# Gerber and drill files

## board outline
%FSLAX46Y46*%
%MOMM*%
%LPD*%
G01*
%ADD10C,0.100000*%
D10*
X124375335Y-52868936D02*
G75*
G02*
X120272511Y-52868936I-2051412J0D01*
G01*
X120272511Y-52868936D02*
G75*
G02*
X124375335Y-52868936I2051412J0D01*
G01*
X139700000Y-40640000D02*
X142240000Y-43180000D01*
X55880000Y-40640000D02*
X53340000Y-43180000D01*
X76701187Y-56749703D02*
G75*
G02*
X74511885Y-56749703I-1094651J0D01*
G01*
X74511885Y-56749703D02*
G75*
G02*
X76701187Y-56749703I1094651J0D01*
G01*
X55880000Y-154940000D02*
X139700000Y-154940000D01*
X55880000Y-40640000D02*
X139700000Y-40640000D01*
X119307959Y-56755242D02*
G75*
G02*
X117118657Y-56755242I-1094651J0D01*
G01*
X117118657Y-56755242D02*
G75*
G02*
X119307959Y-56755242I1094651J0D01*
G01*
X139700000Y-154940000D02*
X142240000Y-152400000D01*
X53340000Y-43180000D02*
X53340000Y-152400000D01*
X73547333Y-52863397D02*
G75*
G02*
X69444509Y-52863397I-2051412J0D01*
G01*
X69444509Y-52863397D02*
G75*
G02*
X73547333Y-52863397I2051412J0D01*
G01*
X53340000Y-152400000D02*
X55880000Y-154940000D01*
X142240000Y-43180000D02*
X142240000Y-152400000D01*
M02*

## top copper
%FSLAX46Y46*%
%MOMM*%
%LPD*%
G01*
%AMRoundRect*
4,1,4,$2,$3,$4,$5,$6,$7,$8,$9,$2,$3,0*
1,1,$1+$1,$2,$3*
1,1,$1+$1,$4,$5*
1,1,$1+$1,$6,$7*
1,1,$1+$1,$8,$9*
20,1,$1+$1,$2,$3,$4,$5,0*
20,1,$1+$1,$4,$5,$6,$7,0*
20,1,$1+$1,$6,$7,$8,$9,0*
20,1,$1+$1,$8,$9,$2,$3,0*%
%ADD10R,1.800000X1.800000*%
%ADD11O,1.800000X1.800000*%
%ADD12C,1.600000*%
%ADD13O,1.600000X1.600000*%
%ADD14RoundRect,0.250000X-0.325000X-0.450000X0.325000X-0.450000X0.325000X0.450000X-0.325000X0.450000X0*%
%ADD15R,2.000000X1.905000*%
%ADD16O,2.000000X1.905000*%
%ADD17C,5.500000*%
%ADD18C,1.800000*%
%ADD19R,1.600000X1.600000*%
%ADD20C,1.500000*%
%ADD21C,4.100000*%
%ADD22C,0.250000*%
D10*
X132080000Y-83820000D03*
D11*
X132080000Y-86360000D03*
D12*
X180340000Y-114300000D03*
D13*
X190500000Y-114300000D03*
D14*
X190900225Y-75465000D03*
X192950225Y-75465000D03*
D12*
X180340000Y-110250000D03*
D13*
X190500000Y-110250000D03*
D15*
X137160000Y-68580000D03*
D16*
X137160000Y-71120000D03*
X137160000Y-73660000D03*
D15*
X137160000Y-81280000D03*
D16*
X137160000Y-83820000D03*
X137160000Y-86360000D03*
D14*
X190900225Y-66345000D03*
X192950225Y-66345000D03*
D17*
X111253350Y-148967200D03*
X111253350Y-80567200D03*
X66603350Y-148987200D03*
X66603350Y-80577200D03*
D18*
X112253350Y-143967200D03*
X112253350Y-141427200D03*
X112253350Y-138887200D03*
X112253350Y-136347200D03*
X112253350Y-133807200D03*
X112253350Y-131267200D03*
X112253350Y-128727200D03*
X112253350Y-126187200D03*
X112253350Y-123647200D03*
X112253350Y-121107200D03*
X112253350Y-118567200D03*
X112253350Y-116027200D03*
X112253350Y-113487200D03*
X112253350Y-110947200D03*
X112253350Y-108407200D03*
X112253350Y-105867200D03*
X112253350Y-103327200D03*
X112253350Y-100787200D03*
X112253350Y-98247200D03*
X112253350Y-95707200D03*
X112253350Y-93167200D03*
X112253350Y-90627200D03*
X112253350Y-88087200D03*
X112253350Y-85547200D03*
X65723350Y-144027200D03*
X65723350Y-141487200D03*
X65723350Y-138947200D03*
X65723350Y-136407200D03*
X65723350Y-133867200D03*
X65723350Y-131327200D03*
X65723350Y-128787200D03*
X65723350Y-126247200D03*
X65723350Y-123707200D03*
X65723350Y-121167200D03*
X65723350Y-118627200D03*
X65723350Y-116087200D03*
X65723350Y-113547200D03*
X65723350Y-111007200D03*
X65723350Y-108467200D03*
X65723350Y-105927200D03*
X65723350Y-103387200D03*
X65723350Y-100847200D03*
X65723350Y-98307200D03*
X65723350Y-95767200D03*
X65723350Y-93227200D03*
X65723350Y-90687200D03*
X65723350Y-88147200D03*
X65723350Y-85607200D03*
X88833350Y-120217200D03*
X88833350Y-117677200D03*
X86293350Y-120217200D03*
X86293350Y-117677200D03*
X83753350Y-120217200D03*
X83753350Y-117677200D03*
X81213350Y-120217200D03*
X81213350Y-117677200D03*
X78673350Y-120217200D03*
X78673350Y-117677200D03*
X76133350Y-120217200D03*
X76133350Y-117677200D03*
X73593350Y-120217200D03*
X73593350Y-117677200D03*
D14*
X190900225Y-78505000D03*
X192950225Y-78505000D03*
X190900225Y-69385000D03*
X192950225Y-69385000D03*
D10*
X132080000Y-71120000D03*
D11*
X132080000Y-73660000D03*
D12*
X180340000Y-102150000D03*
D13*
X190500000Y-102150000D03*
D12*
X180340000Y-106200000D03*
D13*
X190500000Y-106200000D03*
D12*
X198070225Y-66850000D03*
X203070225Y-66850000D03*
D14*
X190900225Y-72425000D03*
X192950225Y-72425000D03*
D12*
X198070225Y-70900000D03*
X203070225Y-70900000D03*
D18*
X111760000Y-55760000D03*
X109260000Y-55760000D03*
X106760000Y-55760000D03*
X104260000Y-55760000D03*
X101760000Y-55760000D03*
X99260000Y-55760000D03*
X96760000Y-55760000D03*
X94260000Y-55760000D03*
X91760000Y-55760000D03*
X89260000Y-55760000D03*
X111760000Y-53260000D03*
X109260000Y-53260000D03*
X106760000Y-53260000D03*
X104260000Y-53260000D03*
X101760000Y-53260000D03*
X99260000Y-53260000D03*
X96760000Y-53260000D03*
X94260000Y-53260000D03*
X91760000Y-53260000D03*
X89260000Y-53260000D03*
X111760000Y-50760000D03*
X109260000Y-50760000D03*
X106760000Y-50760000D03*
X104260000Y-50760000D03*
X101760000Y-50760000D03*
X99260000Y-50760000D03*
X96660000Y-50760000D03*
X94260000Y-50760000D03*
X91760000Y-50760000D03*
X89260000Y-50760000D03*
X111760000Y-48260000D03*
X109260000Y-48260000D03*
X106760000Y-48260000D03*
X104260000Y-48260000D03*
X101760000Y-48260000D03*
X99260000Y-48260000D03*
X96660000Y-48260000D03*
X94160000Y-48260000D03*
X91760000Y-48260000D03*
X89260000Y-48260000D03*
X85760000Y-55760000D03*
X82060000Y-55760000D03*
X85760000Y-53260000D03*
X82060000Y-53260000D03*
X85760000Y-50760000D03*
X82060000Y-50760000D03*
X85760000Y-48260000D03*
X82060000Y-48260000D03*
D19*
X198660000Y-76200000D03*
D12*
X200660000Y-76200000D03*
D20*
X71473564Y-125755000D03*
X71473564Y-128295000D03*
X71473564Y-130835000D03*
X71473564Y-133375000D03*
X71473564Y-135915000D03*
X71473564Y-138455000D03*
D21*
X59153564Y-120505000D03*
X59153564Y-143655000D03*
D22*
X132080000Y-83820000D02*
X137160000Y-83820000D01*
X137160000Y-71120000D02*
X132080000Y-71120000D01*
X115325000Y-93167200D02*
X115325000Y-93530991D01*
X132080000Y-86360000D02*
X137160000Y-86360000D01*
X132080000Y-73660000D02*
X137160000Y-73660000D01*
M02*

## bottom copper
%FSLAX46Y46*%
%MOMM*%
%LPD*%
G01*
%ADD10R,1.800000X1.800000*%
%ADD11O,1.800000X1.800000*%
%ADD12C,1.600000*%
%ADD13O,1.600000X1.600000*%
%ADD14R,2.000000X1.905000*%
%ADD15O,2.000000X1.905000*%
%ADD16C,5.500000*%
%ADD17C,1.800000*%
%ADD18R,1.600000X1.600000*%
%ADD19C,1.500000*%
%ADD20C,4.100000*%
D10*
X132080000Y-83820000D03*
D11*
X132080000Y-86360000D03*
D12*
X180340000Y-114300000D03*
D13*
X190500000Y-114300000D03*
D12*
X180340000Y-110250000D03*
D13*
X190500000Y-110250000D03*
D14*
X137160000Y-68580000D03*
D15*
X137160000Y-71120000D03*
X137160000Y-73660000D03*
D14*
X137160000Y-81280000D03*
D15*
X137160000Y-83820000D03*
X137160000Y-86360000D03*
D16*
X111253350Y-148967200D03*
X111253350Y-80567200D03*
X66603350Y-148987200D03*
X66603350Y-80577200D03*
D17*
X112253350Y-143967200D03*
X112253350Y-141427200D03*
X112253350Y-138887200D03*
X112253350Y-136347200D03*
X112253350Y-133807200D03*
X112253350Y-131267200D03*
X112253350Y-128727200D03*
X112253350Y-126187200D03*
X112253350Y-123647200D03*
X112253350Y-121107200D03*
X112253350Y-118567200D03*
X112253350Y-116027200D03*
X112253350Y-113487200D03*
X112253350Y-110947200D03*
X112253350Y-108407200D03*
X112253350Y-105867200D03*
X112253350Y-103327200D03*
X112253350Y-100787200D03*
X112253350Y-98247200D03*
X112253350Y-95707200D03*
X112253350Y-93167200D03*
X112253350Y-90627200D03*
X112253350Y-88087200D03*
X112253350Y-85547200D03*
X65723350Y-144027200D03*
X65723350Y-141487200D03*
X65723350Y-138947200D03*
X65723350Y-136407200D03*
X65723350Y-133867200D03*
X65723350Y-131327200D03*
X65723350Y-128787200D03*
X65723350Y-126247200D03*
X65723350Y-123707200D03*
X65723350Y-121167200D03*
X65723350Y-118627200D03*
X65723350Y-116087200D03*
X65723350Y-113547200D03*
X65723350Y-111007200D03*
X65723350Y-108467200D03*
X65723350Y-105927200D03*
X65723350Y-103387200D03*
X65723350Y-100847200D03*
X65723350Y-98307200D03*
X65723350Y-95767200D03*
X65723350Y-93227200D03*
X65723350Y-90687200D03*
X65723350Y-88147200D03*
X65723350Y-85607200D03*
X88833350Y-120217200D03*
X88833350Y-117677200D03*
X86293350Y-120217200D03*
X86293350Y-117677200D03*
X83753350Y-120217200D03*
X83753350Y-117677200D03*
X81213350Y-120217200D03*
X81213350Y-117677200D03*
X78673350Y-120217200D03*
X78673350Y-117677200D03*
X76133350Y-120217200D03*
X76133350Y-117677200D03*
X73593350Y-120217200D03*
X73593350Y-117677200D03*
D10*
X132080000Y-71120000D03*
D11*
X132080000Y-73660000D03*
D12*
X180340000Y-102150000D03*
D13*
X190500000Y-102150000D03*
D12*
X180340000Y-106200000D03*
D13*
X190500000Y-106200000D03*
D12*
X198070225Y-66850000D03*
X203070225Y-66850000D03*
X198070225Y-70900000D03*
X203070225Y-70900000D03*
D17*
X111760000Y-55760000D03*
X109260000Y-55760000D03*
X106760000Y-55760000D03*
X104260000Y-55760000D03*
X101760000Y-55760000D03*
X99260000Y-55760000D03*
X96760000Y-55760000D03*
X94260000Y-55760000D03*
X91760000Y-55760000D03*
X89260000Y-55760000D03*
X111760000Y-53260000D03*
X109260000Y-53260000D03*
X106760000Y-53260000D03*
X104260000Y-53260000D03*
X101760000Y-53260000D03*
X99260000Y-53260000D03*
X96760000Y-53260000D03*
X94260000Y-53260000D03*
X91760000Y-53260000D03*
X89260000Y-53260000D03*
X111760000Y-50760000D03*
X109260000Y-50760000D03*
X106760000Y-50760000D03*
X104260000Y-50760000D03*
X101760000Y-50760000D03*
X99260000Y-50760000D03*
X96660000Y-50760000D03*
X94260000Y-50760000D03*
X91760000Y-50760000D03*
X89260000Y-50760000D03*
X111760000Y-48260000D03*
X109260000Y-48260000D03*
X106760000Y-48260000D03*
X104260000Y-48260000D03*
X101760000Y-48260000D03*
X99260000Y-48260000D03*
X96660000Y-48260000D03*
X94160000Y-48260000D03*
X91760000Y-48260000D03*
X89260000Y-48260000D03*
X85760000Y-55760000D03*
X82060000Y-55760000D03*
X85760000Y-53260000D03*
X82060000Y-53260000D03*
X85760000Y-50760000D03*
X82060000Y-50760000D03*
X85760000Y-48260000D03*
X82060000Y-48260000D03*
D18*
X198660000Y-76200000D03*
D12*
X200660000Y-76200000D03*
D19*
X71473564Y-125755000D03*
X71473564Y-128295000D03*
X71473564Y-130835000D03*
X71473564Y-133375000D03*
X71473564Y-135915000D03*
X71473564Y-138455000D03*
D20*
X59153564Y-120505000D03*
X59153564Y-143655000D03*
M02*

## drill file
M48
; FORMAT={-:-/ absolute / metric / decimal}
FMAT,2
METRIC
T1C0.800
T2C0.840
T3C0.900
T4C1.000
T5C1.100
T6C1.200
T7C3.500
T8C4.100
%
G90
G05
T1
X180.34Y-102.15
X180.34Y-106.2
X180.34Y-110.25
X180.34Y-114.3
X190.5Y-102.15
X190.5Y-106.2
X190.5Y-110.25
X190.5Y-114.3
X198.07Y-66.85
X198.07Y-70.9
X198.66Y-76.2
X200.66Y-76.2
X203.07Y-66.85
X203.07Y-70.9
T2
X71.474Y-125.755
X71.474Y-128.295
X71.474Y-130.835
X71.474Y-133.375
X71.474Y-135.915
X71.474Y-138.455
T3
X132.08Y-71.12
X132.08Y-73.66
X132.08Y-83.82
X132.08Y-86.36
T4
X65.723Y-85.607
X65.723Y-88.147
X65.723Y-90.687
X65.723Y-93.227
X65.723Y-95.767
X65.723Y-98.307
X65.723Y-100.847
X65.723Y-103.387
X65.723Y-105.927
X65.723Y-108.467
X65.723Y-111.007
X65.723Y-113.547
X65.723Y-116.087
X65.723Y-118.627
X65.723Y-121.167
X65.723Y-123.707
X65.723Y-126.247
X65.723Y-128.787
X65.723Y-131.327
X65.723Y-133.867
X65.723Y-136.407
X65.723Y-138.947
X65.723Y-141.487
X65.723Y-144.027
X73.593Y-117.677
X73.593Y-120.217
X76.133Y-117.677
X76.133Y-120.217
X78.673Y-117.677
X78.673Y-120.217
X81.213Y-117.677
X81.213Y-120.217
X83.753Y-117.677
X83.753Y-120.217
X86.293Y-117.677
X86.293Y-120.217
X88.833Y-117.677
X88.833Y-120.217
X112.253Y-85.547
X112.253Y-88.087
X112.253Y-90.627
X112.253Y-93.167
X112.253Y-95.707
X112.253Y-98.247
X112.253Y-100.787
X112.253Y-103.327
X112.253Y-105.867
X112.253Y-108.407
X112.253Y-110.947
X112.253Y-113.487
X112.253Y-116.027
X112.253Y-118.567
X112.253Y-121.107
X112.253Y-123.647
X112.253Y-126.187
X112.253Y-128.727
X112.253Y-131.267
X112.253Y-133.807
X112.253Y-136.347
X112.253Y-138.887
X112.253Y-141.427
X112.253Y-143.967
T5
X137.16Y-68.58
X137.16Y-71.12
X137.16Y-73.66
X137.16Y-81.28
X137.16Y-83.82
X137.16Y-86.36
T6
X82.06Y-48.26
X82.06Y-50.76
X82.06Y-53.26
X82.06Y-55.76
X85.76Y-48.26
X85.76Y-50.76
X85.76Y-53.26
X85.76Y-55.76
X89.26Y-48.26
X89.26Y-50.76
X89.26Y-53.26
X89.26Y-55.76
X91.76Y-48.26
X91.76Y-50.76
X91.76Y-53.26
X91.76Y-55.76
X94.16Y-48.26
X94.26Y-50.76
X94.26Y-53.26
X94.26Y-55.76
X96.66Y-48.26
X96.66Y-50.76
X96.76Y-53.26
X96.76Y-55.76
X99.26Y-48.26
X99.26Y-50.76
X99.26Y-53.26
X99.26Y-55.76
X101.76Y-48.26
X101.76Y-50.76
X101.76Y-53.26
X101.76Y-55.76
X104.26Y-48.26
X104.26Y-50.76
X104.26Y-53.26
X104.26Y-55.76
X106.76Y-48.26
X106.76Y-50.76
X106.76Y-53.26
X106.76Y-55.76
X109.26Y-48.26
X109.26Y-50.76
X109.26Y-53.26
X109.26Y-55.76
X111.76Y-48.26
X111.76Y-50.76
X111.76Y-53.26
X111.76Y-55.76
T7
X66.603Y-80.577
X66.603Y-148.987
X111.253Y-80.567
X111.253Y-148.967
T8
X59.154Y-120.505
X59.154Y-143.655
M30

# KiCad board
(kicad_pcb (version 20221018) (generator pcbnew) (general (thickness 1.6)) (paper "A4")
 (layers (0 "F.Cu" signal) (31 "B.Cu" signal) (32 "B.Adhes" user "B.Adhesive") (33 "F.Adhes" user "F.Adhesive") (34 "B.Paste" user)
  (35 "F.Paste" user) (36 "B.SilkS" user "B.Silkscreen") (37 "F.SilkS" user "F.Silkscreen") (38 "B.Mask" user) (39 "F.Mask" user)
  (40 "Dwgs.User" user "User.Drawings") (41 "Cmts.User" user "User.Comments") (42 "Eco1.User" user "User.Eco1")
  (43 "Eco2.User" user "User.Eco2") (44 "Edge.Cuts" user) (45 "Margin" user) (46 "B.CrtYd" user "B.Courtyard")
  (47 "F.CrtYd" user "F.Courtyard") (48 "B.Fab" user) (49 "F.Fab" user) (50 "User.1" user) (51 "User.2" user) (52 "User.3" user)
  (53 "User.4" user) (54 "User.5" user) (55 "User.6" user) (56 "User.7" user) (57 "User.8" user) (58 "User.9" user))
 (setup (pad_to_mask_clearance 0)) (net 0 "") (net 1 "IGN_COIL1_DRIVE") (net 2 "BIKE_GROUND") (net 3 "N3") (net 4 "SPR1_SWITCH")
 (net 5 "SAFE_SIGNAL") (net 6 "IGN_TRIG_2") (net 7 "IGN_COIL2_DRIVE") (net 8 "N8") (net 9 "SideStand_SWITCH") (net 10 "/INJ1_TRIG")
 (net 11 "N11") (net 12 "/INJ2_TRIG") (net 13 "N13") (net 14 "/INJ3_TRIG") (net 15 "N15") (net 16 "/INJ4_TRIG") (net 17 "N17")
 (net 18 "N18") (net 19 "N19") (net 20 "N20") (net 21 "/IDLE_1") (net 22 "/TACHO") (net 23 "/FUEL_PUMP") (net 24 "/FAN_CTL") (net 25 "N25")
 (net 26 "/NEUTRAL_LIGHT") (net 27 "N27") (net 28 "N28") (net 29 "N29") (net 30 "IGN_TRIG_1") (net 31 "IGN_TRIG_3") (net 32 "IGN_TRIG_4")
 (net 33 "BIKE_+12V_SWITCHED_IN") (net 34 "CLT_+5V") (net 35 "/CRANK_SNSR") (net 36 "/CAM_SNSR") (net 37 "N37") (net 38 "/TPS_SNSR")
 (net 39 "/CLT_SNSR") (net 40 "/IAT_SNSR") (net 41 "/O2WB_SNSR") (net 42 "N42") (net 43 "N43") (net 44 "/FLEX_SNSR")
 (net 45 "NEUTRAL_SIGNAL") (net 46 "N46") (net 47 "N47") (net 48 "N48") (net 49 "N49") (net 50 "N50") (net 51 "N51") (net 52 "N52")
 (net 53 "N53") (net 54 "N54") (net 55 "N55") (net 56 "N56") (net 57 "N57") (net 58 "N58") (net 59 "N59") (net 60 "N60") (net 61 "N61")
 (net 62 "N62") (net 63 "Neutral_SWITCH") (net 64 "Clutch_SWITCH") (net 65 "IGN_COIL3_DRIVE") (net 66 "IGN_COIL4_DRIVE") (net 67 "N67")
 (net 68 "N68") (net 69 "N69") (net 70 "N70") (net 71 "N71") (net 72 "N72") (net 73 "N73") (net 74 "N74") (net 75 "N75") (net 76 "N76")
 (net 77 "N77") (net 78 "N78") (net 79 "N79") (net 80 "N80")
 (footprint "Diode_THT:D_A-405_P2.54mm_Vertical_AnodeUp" (layer "F.Cu") (at 132.08 83.82 -90)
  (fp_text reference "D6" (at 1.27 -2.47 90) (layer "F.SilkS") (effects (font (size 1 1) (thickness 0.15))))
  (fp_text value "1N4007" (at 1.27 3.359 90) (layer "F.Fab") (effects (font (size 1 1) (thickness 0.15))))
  (pad "1" thru_hole rect (at 0 0 270) (size 1.8 1.8) (drill 0.9) (layers "*.Cu" "*.Mask") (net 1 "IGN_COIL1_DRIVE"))
  (pad "2" thru_hole oval (at 2.54 0 270) (size 1.8 1.8) (drill 0.9) (layers "*.Cu" "*.Mask") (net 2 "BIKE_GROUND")))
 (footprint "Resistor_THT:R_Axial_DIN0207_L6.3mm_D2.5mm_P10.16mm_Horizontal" (layer "F.Cu") (at 180.34 114.3)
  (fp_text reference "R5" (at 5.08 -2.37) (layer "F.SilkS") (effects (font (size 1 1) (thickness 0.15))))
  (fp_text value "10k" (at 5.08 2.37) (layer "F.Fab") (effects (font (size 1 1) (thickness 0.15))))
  (pad "1" thru_hole circle (at 0 0) (size 1.6 1.6) (drill 0.8) (layers "*.Cu" "*.Mask") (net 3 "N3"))
  (pad "2" thru_hole oval (at 10.16 0) (size 1.6 1.6) (drill 0.8) (layers "*.Cu" "*.Mask") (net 2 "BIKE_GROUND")))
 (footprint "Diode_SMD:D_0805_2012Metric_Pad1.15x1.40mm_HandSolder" (layer "F.Cu") (at 191.925225 75.465)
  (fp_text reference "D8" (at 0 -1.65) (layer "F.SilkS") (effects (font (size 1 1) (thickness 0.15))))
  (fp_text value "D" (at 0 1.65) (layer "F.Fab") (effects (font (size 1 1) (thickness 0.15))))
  (pad "1" smd roundrect (at -1.025 0) (size 1.15 1.4) (layers "F.Cu" "F.Paste" "F.Mask") (roundrect_rratio 0.217391) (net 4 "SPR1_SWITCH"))
  (pad "2" smd roundrect (at 1.025 0) (size 1.15 1.4) (layers "F.Cu" "F.Paste" "F.Mask") (roundrect_rratio 0.217391) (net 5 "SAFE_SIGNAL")))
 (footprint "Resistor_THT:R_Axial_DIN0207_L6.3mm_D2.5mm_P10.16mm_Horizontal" (layer "F.Cu") (at 180.34 110.25)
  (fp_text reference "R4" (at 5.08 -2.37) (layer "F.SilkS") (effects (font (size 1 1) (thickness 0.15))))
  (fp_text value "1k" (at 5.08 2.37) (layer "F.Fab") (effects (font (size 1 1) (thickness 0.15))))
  (pad "1" thru_hole circle (at 0 0) (size 1.6 1.6) (drill 0.8) (layers "*.Cu" "*.Mask") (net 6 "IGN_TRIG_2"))
  (pad "2" thru_hole oval (at 10.16 0) (size 1.6 1.6) (drill 0.8) (layers "*.Cu" "*.Mask") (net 3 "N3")))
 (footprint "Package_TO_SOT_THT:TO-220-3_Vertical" (layer "F.Cu") (at 137.16 68.58 -90)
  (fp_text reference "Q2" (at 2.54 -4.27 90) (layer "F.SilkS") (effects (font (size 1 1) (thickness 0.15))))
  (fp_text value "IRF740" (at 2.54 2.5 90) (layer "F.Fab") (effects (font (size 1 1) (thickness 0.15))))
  (pad "1" thru_hole rect (at 0 0 270) (size 1.905 2) (drill 1.1) (layers "*.Cu" "*.Mask") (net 3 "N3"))
  (pad "2" thru_hole oval (at 2.54 0 270) (size 1.905 2) (drill 1.1) (layers "*.Cu" "*.Mask") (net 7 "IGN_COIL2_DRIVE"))
  (pad "3" thru_hole oval (at 5.08 0 270) (size 1.905 2) (drill 1.1) (layers "*.Cu" "*.Mask") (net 2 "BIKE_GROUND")))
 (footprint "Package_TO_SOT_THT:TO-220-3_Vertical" (layer "F.Cu") (at 137.16 81.28 -90)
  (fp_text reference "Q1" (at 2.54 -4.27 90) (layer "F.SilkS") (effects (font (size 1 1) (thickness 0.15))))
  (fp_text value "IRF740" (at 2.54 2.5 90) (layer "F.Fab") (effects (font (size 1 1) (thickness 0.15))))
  (pad "1" thru_hole rect (at 0 0 270) (size 1.905 2) (drill 1.1) (layers "*.Cu" "*.Mask") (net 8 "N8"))
  (pad "2" thru_hole oval (at 2.54 0 270) (size 1.905 2) (drill 1.1) (layers "*.Cu" "*.Mask") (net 1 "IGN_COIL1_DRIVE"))
  (pad "3" thru_hole oval (at 5.08 0 270) (size 1.905 2) (drill 1.1) (layers "*.Cu" "*.Mask") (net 2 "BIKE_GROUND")))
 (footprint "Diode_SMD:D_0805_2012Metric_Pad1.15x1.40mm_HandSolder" (layer "F.Cu") (at 191.925225 66.345)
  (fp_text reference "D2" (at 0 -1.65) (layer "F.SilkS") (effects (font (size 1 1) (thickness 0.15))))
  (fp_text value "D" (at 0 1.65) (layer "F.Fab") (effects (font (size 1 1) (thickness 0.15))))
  (pad "1" smd roundrect (at -1.025 0) (size 1.15 1.4) (layers "F.Cu" "F.Paste" "F.Mask") (roundrect_rratio 0.217391)
   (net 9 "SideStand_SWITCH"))
  (pad "2" smd roundrect (at 1.025 0) (size 1.15 1.4) (layers "F.Cu" "F.Paste" "F.Mask") (roundrect_rratio 0.217391) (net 5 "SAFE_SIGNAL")))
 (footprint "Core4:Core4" (layer "F.Cu") (at 112.25335 143.9672 180)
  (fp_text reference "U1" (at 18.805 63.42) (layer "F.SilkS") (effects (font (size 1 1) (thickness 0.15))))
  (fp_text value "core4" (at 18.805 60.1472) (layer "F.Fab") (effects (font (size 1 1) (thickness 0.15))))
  (pad "" thru_hole circle (at 1 -5 180) (size 5.5 5.5) (drill 3.5) (layers "*.Cu" "*.Mask"))
  (pad "" thru_hole circle (at 1 63.4 180) (size 5.5 5.5) (drill 3.5) (layers "*.Cu" "*.Mask"))
  (pad "" thru_hole circle (at 45.65 -5.02 180) (size 5.5 5.5) (drill 3.5) (layers "*.Cu" "*.Mask"))
  (pad "" thru_hole circle (at 45.65 63.39 180) (size 5.5 5.5) (drill 3.5) (layers "*.Cu" "*.Mask"))
  (pad "1" thru_hole circle (at 0 0 180) (size 1.8 1.8) (drill 1) (layers "*.Cu" "*.Mask") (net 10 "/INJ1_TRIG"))
  (pad "2" thru_hole circle (at 0 2.54 180) (size 1.8 1.8) (drill 1) (layers "*.Cu" "*.Mask") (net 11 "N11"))
  (pad "3" thru_hole circle (at 0 5.08 180) (size 1.8 1.8) (drill 1) (layers "*.Cu" "*.Mask") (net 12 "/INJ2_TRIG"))
  (pad "4" thru_hole circle (at 0 7.62 180) (size 1.8 1.8) (drill 1) (layers "*.Cu" "*.Mask") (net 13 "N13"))
  (pad "5" thru_hole circle (at 0 10.16 180) (size 1.8 1.8) (drill 1) (layers "*.Cu" "*.Mask") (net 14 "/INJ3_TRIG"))
  (pad "6" thru_hole circle (at 0 12.7 180) (size 1.8 1.8) (drill 1) (layers "*.Cu" "*.Mask") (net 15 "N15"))
  (pad "7" thru_hole circle (at 0 15.24 180) (size 1.8 1.8) (drill 1) (layers "*.Cu" "*.Mask") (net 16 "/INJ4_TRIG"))
  (pad "8" thru_hole circle (at 0 17.78 180) (size 1.8 1.8) (drill 1) (layers "*.Cu" "*.Mask") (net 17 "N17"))
  (pad "9" thru_hole circle (at 0 20.32 180) (size 1.8 1.8) (drill 1) (layers "*.Cu" "*.Mask") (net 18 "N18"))
  (pad "10" thru_hole circle (at 0 22.86 180) (size 1.8 1.8) (drill 1) (layers "*.Cu" "*.Mask") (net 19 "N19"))
  (pad "11" thru_hole circle (at 0 25.4 180) (size 1.8 1.8) (drill 1) (layers "*.Cu" "*.Mask") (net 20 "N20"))
  (pad "12" thru_hole circle (at 0 27.94 180) (size 1.8 1.8) (drill 1) (layers "*.Cu" "*.Mask") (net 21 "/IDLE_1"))
  (pad "13" thru_hole circle (at 0 30.48 180) (size 1.8 1.8) (drill 1) (layers "*.Cu" "*.Mask") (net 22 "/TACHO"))
  (pad "14" thru_hole circle (at 0 33.02 180) (size 1.8 1.8) (drill 1) (layers "*.Cu" "*.Mask") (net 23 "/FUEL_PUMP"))
  (pad "15" thru_hole circle (at 0 35.56 180) (size 1.8 1.8) (drill 1) (layers "*.Cu" "*.Mask") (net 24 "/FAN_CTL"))
  (pad "16" thru_hole circle (at 0 38.1 180) (size 1.8 1.8) (drill 1) (layers "*.Cu" "*.Mask") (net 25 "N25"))
  (pad "17" thru_hole circle (at 0 40.64 180) (size 1.8 1.8) (drill 1) (layers "*.Cu" "*.Mask") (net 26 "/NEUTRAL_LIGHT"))
  (pad "18" thru_hole circle (at 0 43.18 180) (size 1.8 1.8) (drill 1) (layers "*.Cu" "*.Mask") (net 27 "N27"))
  (pad "19" thru_hole circle (at 0 45.72 180) (size 1.8 1.8) (drill 1) (layers "*.Cu" "*.Mask") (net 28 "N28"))
  (pad "20" thru_hole circle (at 0 48.26 180) (size 1.8 1.8) (drill 1) (layers "*.Cu" "*.Mask") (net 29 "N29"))
  (pad "21" thru_hole circle (at 0 50.8 180) (size 1.8 1.8) (drill 1) (layers "*.Cu" "*.Mask") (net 6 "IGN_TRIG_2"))
  (pad "22" thru_hole circle (at 0 53.34 180) (size 1.8 1.8) (drill 1) (layers "*.Cu" "*.Mask") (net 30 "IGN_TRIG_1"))
  (pad "23" thru_hole circle (at 0 55.88 180) (size 1.8 1.8) (drill 1) (layers "*.Cu" "*.Mask") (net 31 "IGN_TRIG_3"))
  (pad "24" thru_hole circle (at 0 58.42 180) (size 1.8 1.8) (drill 1) (layers "*.Cu" "*.Mask") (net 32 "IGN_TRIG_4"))
  (pad "25" thru_hole circle (at 46.53 -0.06 180) (size 1.8 1.8) (drill 1) (layers "*.Cu" "*.Mask") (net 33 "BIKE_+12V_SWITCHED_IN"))
  (pad "26" thru_hole circle (at 46.53 2.48 180) (size 1.8 1.8) (drill 1) (layers "*.Cu" "*.Mask") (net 2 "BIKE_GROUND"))
  (pad "27" thru_hole circle (at 46.53 5.02 180) (size 1.8 1.8) (drill 1) (layers "*.Cu" "*.Mask") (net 2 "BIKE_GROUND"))
  (pad "28" thru_hole circle (at 46.53 7.56 180) (size 1.8 1.8) (drill 1) (layers "*.Cu" "*.Mask") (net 2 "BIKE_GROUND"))
  (pad "29" thru_hole circle (at 46.53 10.1 180) (size 1.8 1.8) (drill 1) (layers "*.Cu" "*.Mask") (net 2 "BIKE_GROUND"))
  (pad "30" thru_hole circle (at 46.53 12.64 180) (size 1.8 1.8) (drill 1) (layers "*.Cu" "*.Mask") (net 2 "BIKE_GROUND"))
  (pad "31" thru_hole circle (at 46.53 15.18 180) (size 1.8 1.8) (drill 1) (layers "*.Cu" "*.Mask") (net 2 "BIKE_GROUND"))
  (pad "32" thru_hole circle (at 46.53 17.72 180) (size 1.8 1.8) (drill 1) (layers "*.Cu" "*.Mask") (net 2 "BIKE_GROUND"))
  (pad "33" thru_hole circle (at 46.53 20.26 180) (size 1.8 1.8) (drill 1) (layers "*.Cu" "*.Mask") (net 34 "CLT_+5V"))
  (pad "34" thru_hole circle (at 46.53 22.8 180) (size 1.8 1.8) (drill 1) (layers "*.Cu" "*.Mask") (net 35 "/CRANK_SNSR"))
  (pad "35" thru_hole circle (at 46.53 25.34 180) (size 1.8 1.8) (drill 1) (layers "*.Cu" "*.Mask") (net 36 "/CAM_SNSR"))
  (pad "36" thru_hole circle (at 46.53 27.88 180) (size 1.8 1.8) (drill 1) (layers "*.Cu" "*.Mask") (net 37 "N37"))
  (pad "37" thru_hole circle (at 46.53 30.42 180) (size 1.8 1.8) (drill 1) (layers "*.Cu" "*.Mask") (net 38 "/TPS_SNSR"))
  (pad "38" thru_hole circle (at 46.53 32.96 180) (size 1.8 1.8) (drill 1) (layers "*.Cu" "*.Mask") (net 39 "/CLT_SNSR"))
  (pad "39" thru_hole circle (at 46.53 35.5 180) (size 1.8 1.8) (drill 1) (layers "*.Cu" "*.Mask") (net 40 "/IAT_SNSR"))
  (pad "40" thru_hole circle (at 46.53 38.04 180) (size 1.8 1.8) (drill 1) (layers "*.Cu" "*.Mask") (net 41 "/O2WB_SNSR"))
  (pad "41" thru_hole circle (at 46.53 40.58 180) (size 1.8 1.8) (drill 1) (layers "*.Cu" "*.Mask") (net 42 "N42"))
  (pad "42" thru_hole circle (at 46.53 43.12 180) (size 1.8 1.8) (drill 1) (layers "*.Cu" "*.Mask") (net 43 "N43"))
  (pad "43" thru_hole circle (at 46.53 45.66 180) (size 1.8 1.8) (drill 1) (layers "*.Cu" "*.Mask") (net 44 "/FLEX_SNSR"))
  (pad "44" thru_hole circle (at 46.53 48.2 180) (size 1.8 1.8) (drill 1) (layers "*.Cu" "*.Mask") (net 5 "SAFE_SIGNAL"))
  (pad "45" thru_hole circle (at 46.53 50.74 180) (size 1.8 1.8) (drill 1) (layers "*.Cu" "*.Mask") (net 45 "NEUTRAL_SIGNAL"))
  (pad "46" thru_hole circle (at 46.53 53.28 180) (size 1.8 1.8) (drill 1) (layers "*.Cu" "*.Mask") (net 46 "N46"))
  (pad "47" thru_hole circle (at 46.53 55.82 180) (size 1.8 1.8) (drill 1) (layers "*.Cu" "*.Mask") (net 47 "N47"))
  (pad "48" thru_hole circle (at 46.53 58.36 180) (size 1.8 1.8) (drill 1) (layers "*.Cu" "*.Mask") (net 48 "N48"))
  (pad "49" thru_hole circle (at 23.42 23.75 180) (size 1.8 1.8) (drill 1) (layers "*.Cu" "*.Mask") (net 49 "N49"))
  (pad "50" thru_hole circle (at 23.42 26.29 180) (size 1.8 1.8) (drill 1) (layers "*.Cu" "*.Mask") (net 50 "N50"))
  (pad "51" thru_hole circle (at 25.96 23.75 180) (size 1.8 1.8) (drill 1) (layers "*.Cu" "*.Mask") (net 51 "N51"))
  (pad "52" thru_hole circle (at 25.96 26.29 180) (size 1.8 1.8) (drill 1) (layers "*.Cu" "*.Mask") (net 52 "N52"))
  (pad "53" thru_hole circle (at 28.5 23.75 180) (size 1.8 1.8) (drill 1) (layers "*.Cu" "*.Mask") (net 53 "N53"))
  (pad "54" thru_hole circle (at 28.5 26.29 180) (size 1.8 1.8) (drill 1) (layers "*.Cu" "*.Mask") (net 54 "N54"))
  (pad "55" thru_hole circle (at 31.04 23.75 180) (size 1.8 1.8) (drill 1) (layers "*.Cu" "*.Mask") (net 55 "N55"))
  (pad "56" thru_hole circle (at 31.04 26.29 180) (size 1.8 1.8) (drill 1) (layers "*.Cu" "*.Mask") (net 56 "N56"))
  (pad "57" thru_hole circle (at 33.58 23.75 180) (size 1.8 1.8) (drill 1) (layers "*.Cu" "*.Mask") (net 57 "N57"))
  (pad "58" thru_hole circle (at 33.58 26.29 180) (size 1.8 1.8) (drill 1) (layers "*.Cu" "*.Mask") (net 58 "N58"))
  (pad "59" thru_hole circle (at 36.12 23.75 180) (size 1.8 1.8) (drill 1) (layers "*.Cu" "*.Mask") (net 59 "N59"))
  (pad "60" thru_hole circle (at 36.12 26.29 180) (size 1.8 1.8) (drill 1) (layers "*.Cu" "*.Mask") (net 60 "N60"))
  (pad "61" thru_hole circle (at 38.66 23.75 180) (size 1.8 1.8) (drill 1) (layers "*.Cu" "*.Mask") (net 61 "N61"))
  (pad "62" thru_hole circle (at 38.66 26.29 180) (size 1.8 1.8) (drill 1) (layers "*.Cu" "*.Mask") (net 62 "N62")))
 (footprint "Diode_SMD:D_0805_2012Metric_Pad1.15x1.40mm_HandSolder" (layer "F.Cu") (at 191.925225 78.505)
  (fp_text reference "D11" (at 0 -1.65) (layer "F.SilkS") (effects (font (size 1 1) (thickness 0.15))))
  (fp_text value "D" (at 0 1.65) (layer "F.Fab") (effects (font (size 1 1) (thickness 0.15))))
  (pad "1" smd roundrect (at -1.025 0) (size 1.15 1.4) (layers "F.Cu" "F.Paste" "F.Mask") (roundrect_rratio 0.217391) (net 4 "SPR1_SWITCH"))
  (pad "2" smd roundrect (at 1.025 0) (size 1.15 1.4) (layers "F.Cu" "F.Paste" "F.Mask") (roundrect_rratio 0.217391) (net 5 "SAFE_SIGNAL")))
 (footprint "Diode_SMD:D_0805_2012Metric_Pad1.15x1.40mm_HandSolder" (layer "F.Cu") (at 191.925225 69.385)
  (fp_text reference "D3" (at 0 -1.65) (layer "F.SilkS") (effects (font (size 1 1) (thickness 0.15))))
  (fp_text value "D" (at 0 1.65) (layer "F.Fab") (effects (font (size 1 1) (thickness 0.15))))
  (pad "1" smd roundrect (at -1.025 0) (size 1.15 1.4) (layers "F.Cu" "F.Paste" "F.Mask") (roundrect_rratio 0.217391)
   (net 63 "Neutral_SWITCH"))
  (pad "2" smd roundrect (at 1.025 0) (size 1.15 1.4) (layers "F.Cu" "F.Paste" "F.Mask") (roundrect_rratio 0.217391) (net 5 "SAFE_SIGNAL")))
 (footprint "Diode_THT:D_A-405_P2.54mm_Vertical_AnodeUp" (layer "F.Cu") (at 132.08 71.12 -90)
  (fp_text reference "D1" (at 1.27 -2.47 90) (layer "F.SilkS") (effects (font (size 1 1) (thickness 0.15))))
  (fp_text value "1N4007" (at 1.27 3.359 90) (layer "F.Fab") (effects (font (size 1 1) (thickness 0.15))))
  (pad "1" thru_hole rect (at 0 0 270) (size 1.8 1.8) (drill 0.9) (layers "*.Cu" "*.Mask") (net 7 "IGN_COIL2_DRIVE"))
  (pad "2" thru_hole oval (at 2.54 0 270) (size 1.8 1.8) (drill 0.9) (layers "*.Cu" "*.Mask") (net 2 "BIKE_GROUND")))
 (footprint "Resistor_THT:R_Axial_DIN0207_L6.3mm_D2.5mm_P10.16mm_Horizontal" (layer "F.Cu") (at 180.34 102.15)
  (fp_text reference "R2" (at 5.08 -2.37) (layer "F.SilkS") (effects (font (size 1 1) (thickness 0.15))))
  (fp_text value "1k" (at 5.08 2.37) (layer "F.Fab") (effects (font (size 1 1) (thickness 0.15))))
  (pad "1" thru_hole circle (at 0 0) (size 1.6 1.6) (drill 0.8) (layers "*.Cu" "*.Mask") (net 30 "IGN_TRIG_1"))
  (pad "2" thru_hole oval (at 10.16 0) (size 1.6 1.6) (drill 0.8) (layers "*.Cu" "*.Mask") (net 8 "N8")))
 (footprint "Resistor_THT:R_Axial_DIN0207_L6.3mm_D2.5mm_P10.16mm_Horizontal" (layer "F.Cu") (at 180.34 106.2)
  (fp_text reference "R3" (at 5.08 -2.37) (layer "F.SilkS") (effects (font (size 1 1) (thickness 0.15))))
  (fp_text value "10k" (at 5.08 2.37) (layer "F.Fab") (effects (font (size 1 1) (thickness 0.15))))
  (pad "1" thru_hole circle (at 0 0) (size 1.6 1.6) (drill 0.8) (layers "*.Cu" "*.Mask") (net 8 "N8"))
  (pad "2" thru_hole oval (at 10.16 0) (size 1.6 1.6) (drill 0.8) (layers "*.Cu" "*.Mask") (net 2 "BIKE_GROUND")))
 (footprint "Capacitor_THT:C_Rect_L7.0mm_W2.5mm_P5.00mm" (layer "F.Cu") (at 198.070225 66.85)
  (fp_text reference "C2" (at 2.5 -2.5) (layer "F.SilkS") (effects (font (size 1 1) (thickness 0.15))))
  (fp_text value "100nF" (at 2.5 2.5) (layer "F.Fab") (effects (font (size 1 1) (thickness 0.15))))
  (pad "1" thru_hole circle (at 0 0) (size 1.6 1.6) (drill 0.8) (layers "*.Cu" "*.Mask") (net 33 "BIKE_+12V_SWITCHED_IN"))
  (pad "2" thru_hole circle (at 5 0) (size 1.6 1.6) (drill 0.8) (layers "*.Cu" "*.Mask") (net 2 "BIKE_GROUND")))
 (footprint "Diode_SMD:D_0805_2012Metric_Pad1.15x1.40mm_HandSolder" (layer "F.Cu") (at 191.925225 72.425)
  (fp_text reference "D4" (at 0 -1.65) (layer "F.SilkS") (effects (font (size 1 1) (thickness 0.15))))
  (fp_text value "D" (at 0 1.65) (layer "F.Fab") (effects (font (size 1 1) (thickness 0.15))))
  (pad "1" smd roundrect (at -1.025 0) (size 1.15 1.4) (layers "F.Cu" "F.Paste" "F.Mask") (roundrect_rratio 0.217391)
   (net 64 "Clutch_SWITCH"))
  (pad "2" smd roundrect (at 1.025 0) (size 1.15 1.4) (layers "F.Cu" "F.Paste" "F.Mask") (roundrect_rratio 0.217391) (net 5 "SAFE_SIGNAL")))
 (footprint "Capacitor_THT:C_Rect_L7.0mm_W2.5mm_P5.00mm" (layer "F.Cu") (at 198.070225 70.9)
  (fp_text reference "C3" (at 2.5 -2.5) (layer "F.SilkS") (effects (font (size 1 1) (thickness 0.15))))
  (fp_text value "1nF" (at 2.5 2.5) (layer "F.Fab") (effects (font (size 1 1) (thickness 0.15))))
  (pad "1" thru_hole circle (at 0 0) (size 1.6 1.6) (drill 0.8) (layers "*.Cu" "*.Mask") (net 33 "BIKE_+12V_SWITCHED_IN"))
  (pad "2" thru_hole circle (at 5 0) (size 1.6 1.6) (drill 0.8) (layers "*.Cu" "*.Mask") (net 2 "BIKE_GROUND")))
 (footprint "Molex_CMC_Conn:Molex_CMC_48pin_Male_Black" (layer "F.Cu") (at 96.91 40.56 180)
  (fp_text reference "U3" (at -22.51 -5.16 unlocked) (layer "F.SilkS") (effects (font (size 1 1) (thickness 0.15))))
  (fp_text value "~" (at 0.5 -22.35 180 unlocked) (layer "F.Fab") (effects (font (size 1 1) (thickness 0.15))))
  (pad "1" thru_hole circle (at -14.85 -15.2 180) (size 1.8 1.8) (drill 1.2) (layers "*.Cu" "*.Mask") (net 10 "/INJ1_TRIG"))
  (pad "2" thru_hole circle (at -12.35 -15.2 180) (size 1.8 1.8) (drill 1.2) (layers "*.Cu" "*.Mask") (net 12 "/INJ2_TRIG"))
  (pad "3" thru_hole circle (at -9.85 -15.2 180) (size 1.8 1.8) (drill 1.2) (layers "*.Cu" "*.Mask") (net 14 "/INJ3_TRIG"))
  (pad "4" thru_hole circle (at -7.35 -15.2 180) (size 1.8 1.8) (drill 1.2) (layers "*.Cu" "*.Mask") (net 16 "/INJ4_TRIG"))
  (pad "5" thru_hole circle (at -4.85 -15.2 180) (size 1.8 1.8) (drill 1.2) (layers "*.Cu" "*.Mask") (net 1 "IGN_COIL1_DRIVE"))
  (pad "6" thru_hole circle (at -2.35 -15.2 180) (size 1.8 1.8) (drill 1.2) (layers "*.Cu" "*.Mask") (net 7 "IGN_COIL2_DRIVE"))
  (pad "7" thru_hole circle (at 0.15 -15.2 180) (size 1.8 1.8) (drill 1.2) (layers "*.Cu" "*.Mask") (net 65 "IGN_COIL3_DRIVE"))
  (pad "8" thru_hole circle (at 2.65 -15.2 180) (size 1.8 1.8) (drill 1.2) (layers "*.Cu" "*.Mask") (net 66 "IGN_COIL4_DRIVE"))
  (pad "9" thru_hole circle (at 5.15 -15.2 180) (size 1.8 1.8) (drill 1.2) (layers "*.Cu" "*.Mask") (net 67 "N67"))
  (pad "10" thru_hole circle (at 7.65 -15.2 180) (size 1.8 1.8) (drill 1.2) (layers "*.Cu" "*.Mask") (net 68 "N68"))
  (pad "11" thru_hole circle (at -14.85 -12.7 180) (size 1.8 1.8) (drill 1.2) (layers "*.Cu" "*.Mask") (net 33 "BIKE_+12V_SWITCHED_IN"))
  (pad "12" thru_hole circle (at -12.35 -12.7 180) (size 1.8 1.8) (drill 1.2) (layers "*.Cu" "*.Mask") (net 22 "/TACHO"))
  (pad "13" thru_hole circle (at -9.85 -12.7 180) (size 1.8 1.8) (drill 1.2) (layers "*.Cu" "*.Mask") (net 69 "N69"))
  (pad "14" thru_hole circle (at -7.35 -12.7 180) (size 1.8 1.8) (drill 1.2) (layers "*.Cu" "*.Mask") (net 33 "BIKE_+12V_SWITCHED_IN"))
  (pad "15" thru_hole circle (at -4.85 -12.7 180) (size 1.8 1.8) (drill 1.2) (layers "*.Cu" "*.Mask") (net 26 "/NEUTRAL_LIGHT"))
  (pad "16" thru_hole circle (at -2.35 -12.7 180) (size 1.8 1.8) (drill 1.2) (layers "*.Cu" "*.Mask") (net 33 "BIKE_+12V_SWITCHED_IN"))
  (pad "17" thru_hole circle (at 0.15 -12.7 180) (size 1.8 1.8) (drill 1.2) (layers "*.Cu" "*.Mask") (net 33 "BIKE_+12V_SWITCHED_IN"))
  (pad "18" thru_hole circle (at 2.65 -12.7 180) (size 1.8 1.8) (drill 1.2) (layers "*.Cu" "*.Mask") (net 24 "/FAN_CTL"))
  (pad "19" thru_hole circle (at 5.15 -12.7 180) (size 1.8 1.8) (drill 1.2) (layers "*.Cu" "*.Mask") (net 21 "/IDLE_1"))
  (pad "20" thru_hole circle (at 7.65 -12.7 180) (size 1.8 1.8) (drill 1.2) (layers "*.Cu" "*.Mask") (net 23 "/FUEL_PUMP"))
  (pad "21" thru_hole circle (at -14.85 -10.2 180) (size 1.8 1.8) (drill 1.2) (layers "*.Cu" "*.Mask") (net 35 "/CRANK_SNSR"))
  (pad "22" thru_hole circle (at -12.35 -10.2 180) (size 1.8 1.8) (drill 1.2) (layers "*.Cu" "*.Mask") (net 2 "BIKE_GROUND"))
  (pad "23" thru_hole circle (at -9.85 -10.2 180) (size 1.8 1.8) (drill 1.2) (layers "*.Cu" "*.Mask") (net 36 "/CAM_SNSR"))
  (pad "24" thru_hole circle (at -7.35 -10.2 180) (size 1.8 1.8) (drill 1.2) (layers "*.Cu" "*.Mask") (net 2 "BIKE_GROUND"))
  (pad "25" thru_hole circle (at -4.85 -10.2 180) (size 1.8 1.8) (drill 1.2) (layers "*.Cu" "*.Mask") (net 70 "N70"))
  (pad "26" thru_hole circle (at -2.35 -10.2 180) (size 1.8 1.8) (drill 1.2) (layers "*.Cu" "*.Mask") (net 44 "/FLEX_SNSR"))
  (pad "27" thru_hole circle (at 0.25 -10.2 180) (size 1.8 1.8) (drill 1.2) (layers "*.Cu" "*.Mask") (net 41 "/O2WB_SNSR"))
  (pad "28" thru_hole circle (at 2.65 -10.2 180) (size 1.8 1.8) (drill 1.2) (layers "*.Cu" "*.Mask") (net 40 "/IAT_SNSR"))
  (pad "29" thru_hole circle (at 5.15 -10.2 180) (size 1.8 1.8) (drill 1.2) (layers "*.Cu" "*.Mask") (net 39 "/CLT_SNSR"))
  (pad "30" thru_hole circle (at 7.65 -10.2 180) (size 1.8 1.8) (drill 1.2) (layers "*.Cu" "*.Mask") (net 38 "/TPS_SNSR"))
  (pad "31" thru_hole circle (at -14.85 -7.7 180) (size 1.8 1.8) (drill 1.2) (layers "*.Cu" "*.Mask") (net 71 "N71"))
  (pad "32" thru_hole circle (at -12.35 -7.7 180) (size 1.8 1.8) (drill 1.2) (layers "*.Cu" "*.Mask") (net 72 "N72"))
  (pad "33" thru_hole circle (at -9.85 -7.7 180) (size 1.8 1.8) (drill 1.2) (layers "*.Cu" "*.Mask") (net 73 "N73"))
  (pad "34" thru_hole circle (at -7.35 -7.7 180) (size 1.8 1.8) (drill 1.2) (layers "*.Cu" "*.Mask") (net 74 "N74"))
  (pad "35" thru_hole circle (at -4.85 -7.7 180) (size 1.8 1.8) (drill 1.2) (layers "*.Cu" "*.Mask") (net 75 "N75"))
  (pad "36" thru_hole circle (at -2.35 -7.7 180) (size 1.8 1.8) (drill 1.2) (layers "*.Cu" "*.Mask") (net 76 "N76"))
  (pad "37" thru_hole circle (at 0.25 -7.7 180) (size 1.8 1.8) (drill 1.2) (layers "*.Cu" "*.Mask") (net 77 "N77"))
  (pad "38" thru_hole circle (at 2.75 -7.7 180) (size 1.8 1.8) (drill 1.2) (layers "*.Cu" "*.Mask") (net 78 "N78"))
  (pad "39" thru_hole circle (at 5.15 -7.7 180) (size 1.8 1.8) (drill 1.2) (layers "*.Cu" "*.Mask") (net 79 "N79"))
  (pad "40" thru_hole circle (at 7.65 -7.7 180) (size 1.8 1.8) (drill 1.2) (layers "*.Cu" "*.Mask") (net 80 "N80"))
  (pad "41" thru_hole circle (at 11.15 -15.2 180) (size 1.8 1.8) (drill 1.2) (layers "*.Cu" "*.Mask") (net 2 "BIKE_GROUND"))
  (pad "42" thru_hole circle (at 14.85 -15.2 180) (size 1.8 1.8) (drill 1.2) (layers "*.Cu" "*.Mask") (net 2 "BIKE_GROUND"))
  (pad "43" thru_hole circle (at 11.15 -12.7 180) (size 1.8 1.8) (drill 1.2) (layers "*.Cu" "*.Mask") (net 2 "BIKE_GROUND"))
  (pad "44" thru_hole circle (at 14.85 -12.7 180) (size 1.8 1.8) (drill 1.2) (layers "*.Cu" "*.Mask") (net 2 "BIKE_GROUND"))
  (pad "45" thru_hole circle (at 11.15 -10.2 180) (size 1.8 1.8) (drill 1.2) (layers "*.Cu" "*.Mask") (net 2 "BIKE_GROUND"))
  (pad "46" thru_hole circle (at 14.85 -10.2 180) (size 1.8 1.8) (drill 1.2) (layers "*.Cu" "*.Mask") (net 2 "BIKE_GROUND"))
  (pad "47" thru_hole circle (at 11.15 -7.7 180) (size 1.8 1.8) (drill 1.2) (layers "*.Cu" "*.Mask") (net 2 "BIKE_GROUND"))
  (pad "48" thru_hole circle (at 14.85 -7.7 180) (size 1.8 1.8) (drill 1.2) (layers "*.Cu" "*.Mask") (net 33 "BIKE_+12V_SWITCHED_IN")))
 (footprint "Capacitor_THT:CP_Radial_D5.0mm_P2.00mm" (layer "F.Cu") (at 198.66 76.2)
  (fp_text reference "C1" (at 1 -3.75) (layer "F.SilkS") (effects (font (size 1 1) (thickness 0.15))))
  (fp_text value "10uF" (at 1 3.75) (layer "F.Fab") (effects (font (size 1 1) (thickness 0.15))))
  (pad "1" thru_hole rect (at 0 0) (size 1.6 1.6) (drill 0.8) (layers "*.Cu" "*.Mask") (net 33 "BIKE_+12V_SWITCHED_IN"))
  (pad "2" thru_hole circle (at 2 0) (size 1.6 1.6) (drill 0.8) (layers "*.Cu" "*.Mask") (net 2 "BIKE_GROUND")))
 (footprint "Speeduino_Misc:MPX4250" (layer "B.Cu") (at 71.473564 125.755 -90)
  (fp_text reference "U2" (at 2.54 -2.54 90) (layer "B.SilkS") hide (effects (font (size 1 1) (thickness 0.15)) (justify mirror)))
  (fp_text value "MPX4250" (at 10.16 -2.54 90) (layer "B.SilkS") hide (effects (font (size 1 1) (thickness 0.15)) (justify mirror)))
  (pad "1" thru_hole circle (at 0 0 270) (size 1.5 1.5) (drill 0.84) (layers "*.Cu" "*.Mask" "B.SilkS") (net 37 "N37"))
  (pad "2" thru_hole circle (at 2.54 0 270) (size 1.5 1.5) (drill 0.84) (layers "*.Cu" "*.Mask" "B.SilkS") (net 2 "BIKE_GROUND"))
  (pad "3" thru_hole circle (at 5.08 0 270) (size 1.5 1.5) (drill 0.84) (layers "*.Cu" "*.Mask" "B.SilkS") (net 34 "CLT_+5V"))
  (pad "4" thru_hole circle (at 7.62 0 270) (size 1.5 1.5) (drill 0.84) (layers "*.Cu" "*.Mask" "B.SilkS"))
  (pad "5" thru_hole circle (at 10.16 0 270) (size 1.5 1.5) (drill 0.84) (layers "*.Cu" "*.Mask" "B.SilkS"))
  (pad "6" thru_hole circle (at 12.7 0 270) (size 1.5 1.5) (drill 0.84) (layers "*.Cu" "*.Mask" "B.SilkS"))
  (pad "~" thru_hole circle (at -5.25 12.32 270) (size 4.1 4.1) (drill 4.1) (layers "*.Cu" "*.Mask" "B.SilkS"))
  (pad "~" thru_hole circle (at 17.9 12.32 270) (size 4.1 4.1) (drill 4.1) (layers "*.Cu" "*.Mask" "B.SilkS")))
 (gr_circle (center 122.323923 52.868936) (end 123.792734 54.301027) (stroke (width 0.1) (type default)) (fill none) (layer "Edge.Cuts"))
 (gr_line (start 139.7 40.64) (end 142.24 43.18) (stroke (width 0.1) (type default)) (layer "Edge.Cuts"))
 (gr_line (start 55.88 40.64) (end 53.34 43.18) (stroke (width 0.1) (type default)) (layer "Edge.Cuts"))
 (gr_circle (center 75.606536 56.749703) (end 74.769978 57.4557) (stroke (width 0.1) (type default)) (fill none) (layer "Edge.Cuts"))
 (gr_line (start 55.88 154.94) (end 139.7 154.94) (stroke (width 0.1) (type default)) (layer "Edge.Cuts"))
 (gr_line (start 55.88 40.64) (end 139.7 40.64) (stroke (width 0.1) (type default)) (layer "Edge.Cuts"))
 (gr_circle (center 118.213308 56.755242) (end 119.049866 57.461239) (stroke (width 0.1) (type default)) (fill none) (layer "Edge.Cuts"))
 (gr_line (start 139.7 154.94) (end 142.24 152.4) (stroke (width 0.1) (type default)) (layer "Edge.Cuts"))
 (gr_line (start 53.34 43.18) (end 53.34 152.4) (stroke (width 0.1) (type default)) (layer "Edge.Cuts"))
 (gr_circle (center 71.495921 52.863397) (end 70.02711 54.295488) (stroke (width 0.1) (type default)) (fill none) (layer "Edge.Cuts"))
 (gr_line (start 53.34 152.4) (end 55.88 154.94) (stroke (width 0.1) (type default)) (layer "Edge.Cuts"))
 (gr_line (start 142.24 43.18) (end 142.24 152.4) (stroke (width 0.1) (type default)) (layer "Edge.Cuts"))
 (segment (start 132.08 83.82) (end 137.16 83.82) (width 0.25) (layer "F.Cu") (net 1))
 (segment (start 137.16 71.12) (end 132.08 71.12) (width 0.25) (layer "F.Cu") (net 7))
 (segment (start 115.325 93.1672) (end 115.325 93.530991) (width 0.25) (layer "F.Cu") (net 6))
 (segment (start 132.08 86.36) (end 137.16 86.36) (width 0.25) (layer "F.Cu") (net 2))
 (segment (start 132.08 73.66) (end 137.16 73.66) (width 0.25) (layer "F.Cu") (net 2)))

